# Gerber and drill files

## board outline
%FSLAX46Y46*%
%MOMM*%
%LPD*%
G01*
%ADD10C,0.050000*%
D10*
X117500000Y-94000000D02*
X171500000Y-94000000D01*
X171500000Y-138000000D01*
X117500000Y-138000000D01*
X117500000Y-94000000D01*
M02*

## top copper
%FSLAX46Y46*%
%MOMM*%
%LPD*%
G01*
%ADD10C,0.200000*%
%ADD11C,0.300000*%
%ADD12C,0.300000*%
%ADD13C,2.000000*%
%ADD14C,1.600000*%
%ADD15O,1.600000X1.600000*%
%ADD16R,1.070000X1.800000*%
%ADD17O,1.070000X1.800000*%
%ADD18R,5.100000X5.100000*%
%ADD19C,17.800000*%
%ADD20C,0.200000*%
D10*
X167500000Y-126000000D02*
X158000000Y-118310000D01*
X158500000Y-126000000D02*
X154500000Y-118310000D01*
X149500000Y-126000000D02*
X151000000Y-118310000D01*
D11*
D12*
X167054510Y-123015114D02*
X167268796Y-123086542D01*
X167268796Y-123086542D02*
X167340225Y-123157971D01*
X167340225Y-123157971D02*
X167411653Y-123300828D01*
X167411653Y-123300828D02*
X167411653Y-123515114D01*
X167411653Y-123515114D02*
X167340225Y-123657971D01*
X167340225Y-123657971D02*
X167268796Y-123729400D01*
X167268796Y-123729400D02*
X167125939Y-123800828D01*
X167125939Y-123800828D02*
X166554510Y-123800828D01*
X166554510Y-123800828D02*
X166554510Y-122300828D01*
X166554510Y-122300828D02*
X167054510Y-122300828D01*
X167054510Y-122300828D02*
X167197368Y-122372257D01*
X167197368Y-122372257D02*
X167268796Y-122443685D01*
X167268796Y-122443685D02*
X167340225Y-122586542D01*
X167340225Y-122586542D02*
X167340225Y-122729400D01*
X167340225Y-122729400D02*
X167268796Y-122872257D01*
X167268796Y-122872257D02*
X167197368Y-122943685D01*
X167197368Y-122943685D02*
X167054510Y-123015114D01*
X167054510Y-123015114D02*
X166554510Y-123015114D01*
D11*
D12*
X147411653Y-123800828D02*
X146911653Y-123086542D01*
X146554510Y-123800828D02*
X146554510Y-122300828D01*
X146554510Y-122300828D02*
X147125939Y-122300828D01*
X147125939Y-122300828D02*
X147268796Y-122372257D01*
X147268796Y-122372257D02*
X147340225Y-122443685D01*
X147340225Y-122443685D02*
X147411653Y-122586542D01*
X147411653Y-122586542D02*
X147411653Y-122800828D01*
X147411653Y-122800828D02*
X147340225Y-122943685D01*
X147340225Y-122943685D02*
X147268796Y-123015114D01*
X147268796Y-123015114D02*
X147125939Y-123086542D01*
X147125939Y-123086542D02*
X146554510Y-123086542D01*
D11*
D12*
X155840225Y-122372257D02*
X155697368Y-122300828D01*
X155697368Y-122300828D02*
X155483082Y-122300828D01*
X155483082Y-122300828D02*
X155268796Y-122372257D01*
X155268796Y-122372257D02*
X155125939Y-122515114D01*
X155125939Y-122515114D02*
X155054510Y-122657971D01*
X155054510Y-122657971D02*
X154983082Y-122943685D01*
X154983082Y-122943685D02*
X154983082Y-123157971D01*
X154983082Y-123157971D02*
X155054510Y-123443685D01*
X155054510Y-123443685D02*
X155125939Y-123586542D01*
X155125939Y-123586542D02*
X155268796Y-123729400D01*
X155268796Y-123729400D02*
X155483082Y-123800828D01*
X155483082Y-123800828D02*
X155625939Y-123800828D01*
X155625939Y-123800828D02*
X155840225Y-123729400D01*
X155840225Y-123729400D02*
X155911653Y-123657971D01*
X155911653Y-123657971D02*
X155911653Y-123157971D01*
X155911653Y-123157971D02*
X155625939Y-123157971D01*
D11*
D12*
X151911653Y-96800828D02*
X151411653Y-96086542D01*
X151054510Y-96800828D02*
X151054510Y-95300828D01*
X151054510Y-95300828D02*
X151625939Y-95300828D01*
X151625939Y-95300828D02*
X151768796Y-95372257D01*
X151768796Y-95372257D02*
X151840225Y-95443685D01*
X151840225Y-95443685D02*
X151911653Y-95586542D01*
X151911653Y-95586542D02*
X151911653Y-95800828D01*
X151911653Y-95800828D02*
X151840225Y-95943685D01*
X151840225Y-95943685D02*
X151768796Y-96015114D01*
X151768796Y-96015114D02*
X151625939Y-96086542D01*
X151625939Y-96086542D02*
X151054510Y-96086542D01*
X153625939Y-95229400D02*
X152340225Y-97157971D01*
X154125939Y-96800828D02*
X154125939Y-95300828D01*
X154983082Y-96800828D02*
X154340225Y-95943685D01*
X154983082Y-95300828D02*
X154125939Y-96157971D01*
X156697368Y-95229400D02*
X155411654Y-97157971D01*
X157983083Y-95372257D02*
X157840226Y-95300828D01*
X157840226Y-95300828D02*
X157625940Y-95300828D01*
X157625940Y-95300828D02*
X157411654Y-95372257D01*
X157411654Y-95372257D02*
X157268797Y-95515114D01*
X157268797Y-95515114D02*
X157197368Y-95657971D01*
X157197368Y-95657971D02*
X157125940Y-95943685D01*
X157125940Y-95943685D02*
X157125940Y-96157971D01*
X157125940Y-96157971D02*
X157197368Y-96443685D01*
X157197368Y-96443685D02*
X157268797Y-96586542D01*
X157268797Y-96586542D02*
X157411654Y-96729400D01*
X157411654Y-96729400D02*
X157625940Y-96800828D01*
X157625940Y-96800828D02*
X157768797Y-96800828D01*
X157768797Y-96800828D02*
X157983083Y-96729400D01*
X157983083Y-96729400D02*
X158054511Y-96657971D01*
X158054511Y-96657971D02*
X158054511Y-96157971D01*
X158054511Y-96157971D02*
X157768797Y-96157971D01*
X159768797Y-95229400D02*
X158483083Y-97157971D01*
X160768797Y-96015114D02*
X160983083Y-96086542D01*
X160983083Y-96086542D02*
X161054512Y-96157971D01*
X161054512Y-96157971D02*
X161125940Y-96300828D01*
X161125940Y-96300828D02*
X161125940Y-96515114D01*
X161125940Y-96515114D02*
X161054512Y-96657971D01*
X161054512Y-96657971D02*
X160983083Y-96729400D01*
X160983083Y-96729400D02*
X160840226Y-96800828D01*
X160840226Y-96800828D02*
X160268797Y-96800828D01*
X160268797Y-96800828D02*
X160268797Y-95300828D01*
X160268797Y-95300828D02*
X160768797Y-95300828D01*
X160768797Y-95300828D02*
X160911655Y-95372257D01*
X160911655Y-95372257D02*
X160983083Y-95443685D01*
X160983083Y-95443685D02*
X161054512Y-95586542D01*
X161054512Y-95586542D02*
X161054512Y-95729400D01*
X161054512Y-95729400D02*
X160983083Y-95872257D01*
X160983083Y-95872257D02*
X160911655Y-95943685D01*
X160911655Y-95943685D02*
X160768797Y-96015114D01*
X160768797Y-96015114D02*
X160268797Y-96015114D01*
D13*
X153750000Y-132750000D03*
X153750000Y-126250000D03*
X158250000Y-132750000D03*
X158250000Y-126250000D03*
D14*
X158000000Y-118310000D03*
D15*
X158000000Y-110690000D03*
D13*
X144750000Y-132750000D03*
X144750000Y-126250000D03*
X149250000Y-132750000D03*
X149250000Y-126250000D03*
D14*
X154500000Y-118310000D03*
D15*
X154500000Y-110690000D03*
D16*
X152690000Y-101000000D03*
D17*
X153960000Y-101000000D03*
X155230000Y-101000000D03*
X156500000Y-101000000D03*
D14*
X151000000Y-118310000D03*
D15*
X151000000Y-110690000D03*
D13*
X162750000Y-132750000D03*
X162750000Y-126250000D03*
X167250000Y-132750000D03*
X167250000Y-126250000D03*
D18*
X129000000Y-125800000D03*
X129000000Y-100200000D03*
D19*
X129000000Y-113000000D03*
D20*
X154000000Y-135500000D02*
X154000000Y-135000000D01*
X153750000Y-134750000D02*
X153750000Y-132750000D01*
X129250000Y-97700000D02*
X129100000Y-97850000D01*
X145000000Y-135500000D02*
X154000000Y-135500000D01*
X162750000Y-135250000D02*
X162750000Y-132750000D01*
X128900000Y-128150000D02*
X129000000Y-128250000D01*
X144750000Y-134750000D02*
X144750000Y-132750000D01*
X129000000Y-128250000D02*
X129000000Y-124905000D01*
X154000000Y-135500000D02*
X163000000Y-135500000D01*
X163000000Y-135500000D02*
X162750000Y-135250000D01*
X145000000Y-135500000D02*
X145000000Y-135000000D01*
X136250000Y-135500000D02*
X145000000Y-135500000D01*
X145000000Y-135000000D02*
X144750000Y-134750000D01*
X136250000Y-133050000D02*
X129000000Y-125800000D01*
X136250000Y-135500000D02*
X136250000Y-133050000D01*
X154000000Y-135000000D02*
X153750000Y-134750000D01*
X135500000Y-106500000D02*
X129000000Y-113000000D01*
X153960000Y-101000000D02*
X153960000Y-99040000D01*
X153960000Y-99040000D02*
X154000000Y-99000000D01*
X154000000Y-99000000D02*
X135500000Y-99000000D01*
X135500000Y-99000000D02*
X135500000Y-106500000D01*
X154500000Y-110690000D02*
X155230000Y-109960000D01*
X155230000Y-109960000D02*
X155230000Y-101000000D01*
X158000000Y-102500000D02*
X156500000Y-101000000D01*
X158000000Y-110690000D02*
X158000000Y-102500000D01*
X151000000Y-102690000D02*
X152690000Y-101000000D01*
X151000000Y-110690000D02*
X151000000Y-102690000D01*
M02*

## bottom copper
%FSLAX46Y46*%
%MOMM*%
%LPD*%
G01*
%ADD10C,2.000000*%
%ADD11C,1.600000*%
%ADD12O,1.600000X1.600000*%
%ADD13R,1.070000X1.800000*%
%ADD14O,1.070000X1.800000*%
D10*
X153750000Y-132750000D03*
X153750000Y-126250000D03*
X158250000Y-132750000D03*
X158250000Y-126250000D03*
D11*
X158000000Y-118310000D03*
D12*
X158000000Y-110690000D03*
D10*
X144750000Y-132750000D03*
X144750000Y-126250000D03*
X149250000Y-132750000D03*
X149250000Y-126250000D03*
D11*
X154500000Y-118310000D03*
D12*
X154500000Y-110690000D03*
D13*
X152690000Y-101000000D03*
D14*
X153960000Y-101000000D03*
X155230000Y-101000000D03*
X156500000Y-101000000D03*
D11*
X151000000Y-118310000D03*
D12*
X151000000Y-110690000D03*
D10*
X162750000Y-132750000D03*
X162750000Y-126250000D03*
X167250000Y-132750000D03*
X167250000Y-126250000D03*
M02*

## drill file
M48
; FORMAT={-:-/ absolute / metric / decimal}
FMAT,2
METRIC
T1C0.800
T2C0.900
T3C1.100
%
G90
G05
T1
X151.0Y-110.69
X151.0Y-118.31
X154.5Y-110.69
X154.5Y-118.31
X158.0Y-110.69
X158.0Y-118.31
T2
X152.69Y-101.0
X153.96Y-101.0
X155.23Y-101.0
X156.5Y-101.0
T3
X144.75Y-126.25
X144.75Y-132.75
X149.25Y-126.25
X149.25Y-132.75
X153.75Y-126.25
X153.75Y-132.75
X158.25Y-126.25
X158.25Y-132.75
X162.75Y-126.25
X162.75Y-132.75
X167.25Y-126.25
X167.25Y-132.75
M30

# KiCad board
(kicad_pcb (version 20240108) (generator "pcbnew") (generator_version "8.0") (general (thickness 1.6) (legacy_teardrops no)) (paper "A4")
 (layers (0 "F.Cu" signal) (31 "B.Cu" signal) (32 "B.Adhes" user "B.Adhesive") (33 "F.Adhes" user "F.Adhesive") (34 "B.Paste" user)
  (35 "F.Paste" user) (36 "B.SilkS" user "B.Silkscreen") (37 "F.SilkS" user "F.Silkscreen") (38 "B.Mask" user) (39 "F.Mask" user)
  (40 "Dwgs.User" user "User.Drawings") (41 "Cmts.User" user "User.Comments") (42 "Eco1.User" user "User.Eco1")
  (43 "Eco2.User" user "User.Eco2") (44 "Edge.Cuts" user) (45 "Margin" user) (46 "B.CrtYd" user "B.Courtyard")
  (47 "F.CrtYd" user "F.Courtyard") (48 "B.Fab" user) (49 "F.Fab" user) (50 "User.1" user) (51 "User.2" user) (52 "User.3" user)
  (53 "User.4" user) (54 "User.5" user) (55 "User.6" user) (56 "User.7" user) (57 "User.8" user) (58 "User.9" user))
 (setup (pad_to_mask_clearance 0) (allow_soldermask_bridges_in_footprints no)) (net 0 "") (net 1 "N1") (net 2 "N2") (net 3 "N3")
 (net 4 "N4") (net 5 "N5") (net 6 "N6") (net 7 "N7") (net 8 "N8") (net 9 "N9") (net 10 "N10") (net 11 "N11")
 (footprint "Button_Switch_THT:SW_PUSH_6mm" (layer "F.Cu") (at 153.75 132.75 90)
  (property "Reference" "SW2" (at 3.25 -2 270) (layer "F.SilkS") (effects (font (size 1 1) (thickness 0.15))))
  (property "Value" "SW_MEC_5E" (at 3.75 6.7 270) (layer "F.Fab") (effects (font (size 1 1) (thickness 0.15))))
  (pad "1" thru_hole circle (at 0 0 180) (size 2 2) (drill 1.1) (layers "*.Cu" "*.Mask") (remove_unused_layers no) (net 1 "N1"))
  (pad "1" thru_hole circle (at 6.5 0 180) (size 2 2) (drill 1.1) (layers "*.Cu" "*.Mask") (remove_unused_layers no) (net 1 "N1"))
  (pad "2" thru_hole circle (at 0 4.5 180) (size 2 2) (drill 1.1) (layers "*.Cu" "*.Mask") (remove_unused_layers no) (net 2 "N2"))
  (pad "2" thru_hole circle (at 6.5 4.5 180) (size 2 2) (drill 1.1) (layers "*.Cu" "*.Mask") (remove_unused_layers no) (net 2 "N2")))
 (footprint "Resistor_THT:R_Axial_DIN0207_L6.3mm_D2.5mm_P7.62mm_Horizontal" (layer "F.Cu") (at 158 118.31 90)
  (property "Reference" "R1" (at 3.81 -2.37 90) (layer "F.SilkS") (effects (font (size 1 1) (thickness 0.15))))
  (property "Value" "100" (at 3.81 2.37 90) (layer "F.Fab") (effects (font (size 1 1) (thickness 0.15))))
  (pad "1" thru_hole circle (at 0 0 90) (size 1.6 1.6) (drill 0.8) (layers "*.Cu" "*.Mask") (remove_unused_layers no) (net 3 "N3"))
  (pad "2" thru_hole oval (at 7.62 0 90) (size 1.6 1.6) (drill 0.8) (layers "*.Cu" "*.Mask") (remove_unused_layers no) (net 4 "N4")))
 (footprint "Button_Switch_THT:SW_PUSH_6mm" (layer "F.Cu") (at 144.75 132.75 90)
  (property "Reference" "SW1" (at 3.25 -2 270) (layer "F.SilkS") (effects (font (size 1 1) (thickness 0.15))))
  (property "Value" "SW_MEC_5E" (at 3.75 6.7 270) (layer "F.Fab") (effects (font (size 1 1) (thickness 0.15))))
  (pad "1" thru_hole circle (at 0 0 180) (size 2 2) (drill 1.1) (layers "*.Cu" "*.Mask") (remove_unused_layers no) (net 1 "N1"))
  (pad "1" thru_hole circle (at 6.5 0 180) (size 2 2) (drill 1.1) (layers "*.Cu" "*.Mask") (remove_unused_layers no) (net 1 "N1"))
  (pad "2" thru_hole circle (at 0 4.5 180) (size 2 2) (drill 1.1) (layers "*.Cu" "*.Mask") (remove_unused_layers no) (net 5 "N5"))
  (pad "2" thru_hole circle (at 6.5 4.5 180) (size 2 2) (drill 1.1) (layers "*.Cu" "*.Mask") (remove_unused_layers no) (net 5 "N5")))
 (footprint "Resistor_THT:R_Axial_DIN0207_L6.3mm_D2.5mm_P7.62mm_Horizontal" (layer "F.Cu") (at 154.5 118.31 90)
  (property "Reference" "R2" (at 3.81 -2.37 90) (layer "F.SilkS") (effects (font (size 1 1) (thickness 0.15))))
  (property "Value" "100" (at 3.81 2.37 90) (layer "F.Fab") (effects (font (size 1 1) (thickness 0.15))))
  (pad "1" thru_hole circle (at 0 0 90) (size 1.6 1.6) (drill 0.8) (layers "*.Cu" "*.Mask") (remove_unused_layers no) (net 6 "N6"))
  (pad "2" thru_hole oval (at 7.62 0 90) (size 1.6 1.6) (drill 0.8) (layers "*.Cu" "*.Mask") (remove_unused_layers no) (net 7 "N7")))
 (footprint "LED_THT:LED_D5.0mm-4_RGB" (layer "F.Cu") (at 152.69 101)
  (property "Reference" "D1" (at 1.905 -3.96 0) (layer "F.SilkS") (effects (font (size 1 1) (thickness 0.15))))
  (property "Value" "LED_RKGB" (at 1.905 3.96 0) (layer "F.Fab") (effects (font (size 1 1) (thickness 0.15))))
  (pad "1" thru_hole rect (at 0 0) (size 1.07 1.8) (drill 0.9) (layers "*.Cu" "*.Mask") (remove_unused_layers no) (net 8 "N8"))
  (pad "2" thru_hole oval (at 1.27 0) (size 1.07 1.8) (drill 0.9) (layers "*.Cu" "*.Mask") (remove_unused_layers no) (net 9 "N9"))
  (pad "3" thru_hole oval (at 2.54 0) (size 1.07 1.8) (drill 0.9) (layers "*.Cu" "*.Mask") (remove_unused_layers no) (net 7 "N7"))
  (pad "4" thru_hole oval (at 3.81 0) (size 1.07 1.8) (drill 0.9) (layers "*.Cu" "*.Mask") (remove_unused_layers no) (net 4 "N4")))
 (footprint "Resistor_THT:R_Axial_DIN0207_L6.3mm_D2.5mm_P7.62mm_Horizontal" (layer "F.Cu") (at 151 118.31 90)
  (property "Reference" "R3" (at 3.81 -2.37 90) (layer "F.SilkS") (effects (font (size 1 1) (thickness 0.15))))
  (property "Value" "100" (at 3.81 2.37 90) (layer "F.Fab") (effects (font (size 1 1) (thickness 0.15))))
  (pad "1" thru_hole circle (at 0 0 90) (size 1.6 1.6) (drill 0.8) (layers "*.Cu" "*.Mask") (remove_unused_layers no) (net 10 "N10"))
  (pad "2" thru_hole oval (at 7.62 0 90) (size 1.6 1.6) (drill 0.8) (layers "*.Cu" "*.Mask") (remove_unused_layers no) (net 8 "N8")))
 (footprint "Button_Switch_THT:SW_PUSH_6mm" (layer "F.Cu") (at 162.75 132.75 90)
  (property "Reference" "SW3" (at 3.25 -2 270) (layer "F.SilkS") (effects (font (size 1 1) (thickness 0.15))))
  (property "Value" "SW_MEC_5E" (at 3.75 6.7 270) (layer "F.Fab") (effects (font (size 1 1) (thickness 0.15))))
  (pad "1" thru_hole circle (at 0 0 180) (size 2 2) (drill 1.1) (layers "*.Cu" "*.Mask") (remove_unused_layers no) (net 1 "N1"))
  (pad "1" thru_hole circle (at 6.5 0 180) (size 2 2) (drill 1.1) (layers "*.Cu" "*.Mask") (remove_unused_layers no) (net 1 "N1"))
  (pad "2" thru_hole circle (at 0 4.5 180) (size 2 2) (drill 1.1) (layers "*.Cu" "*.Mask") (remove_unused_layers no) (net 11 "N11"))
  (pad "2" thru_hole circle (at 6.5 4.5 180) (size 2 2) (drill 1.1) (layers "*.Cu" "*.Mask") (remove_unused_layers no) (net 11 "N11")))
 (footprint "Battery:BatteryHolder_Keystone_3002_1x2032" (layer "F.Cu") (at 129 113 90)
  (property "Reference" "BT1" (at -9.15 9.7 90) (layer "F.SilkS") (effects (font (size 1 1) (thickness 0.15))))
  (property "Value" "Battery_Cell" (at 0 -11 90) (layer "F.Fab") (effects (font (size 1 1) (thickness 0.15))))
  (pad "1" smd rect (at -12.8 0 90) (size 5.1 5.1) (layers "F.Cu" "F.Paste" "F.Mask") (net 1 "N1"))
  (pad "1" smd rect (at 12.8 0 90) (size 5.1 5.1) (layers "F.Cu" "F.Paste" "F.Mask") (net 1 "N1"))
  (pad "2" smd circle (at 0 0 90) (size 17.8 17.8) (layers "F.Cu" "F.Mask") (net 9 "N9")))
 (gr_line (start 167.5 126) (end 158 118.31) (stroke (width 0.2) (type default)) (layer "F.Cu"))
 (gr_line (start 158.5 126) (end 154.5 118.31) (stroke (width 0.2) (type default)) (layer "F.Cu"))
 (gr_line (start 149.5 126) (end 151 118.31) (stroke (width 0.2) (type default)) (layer "F.Cu"))
 (gr_rect (start 117.5 94) (end 171.5 138) (stroke (width 0.05) (type default)) (fill none) (layer "Edge.Cuts"))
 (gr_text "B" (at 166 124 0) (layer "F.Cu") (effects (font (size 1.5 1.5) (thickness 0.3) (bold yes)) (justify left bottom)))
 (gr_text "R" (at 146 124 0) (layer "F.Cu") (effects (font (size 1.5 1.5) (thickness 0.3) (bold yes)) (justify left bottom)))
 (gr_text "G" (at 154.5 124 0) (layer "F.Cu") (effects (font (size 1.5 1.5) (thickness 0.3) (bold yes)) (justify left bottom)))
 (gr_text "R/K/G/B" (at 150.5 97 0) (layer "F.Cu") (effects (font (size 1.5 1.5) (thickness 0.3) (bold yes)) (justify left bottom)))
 (segment (start 154 135.5) (end 154 135) (width 0.2) (layer "F.Cu") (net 1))
 (segment (start 153.75 134.75) (end 153.75 132.75) (width 0.2) (layer "F.Cu") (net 1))
 (segment (start 129.25 97.7) (end 129.1 97.85) (width 0.2) (layer "F.Cu") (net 1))
 (segment (start 145 135.5) (end 154 135.5) (width 0.2) (layer "F.Cu") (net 1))
 (segment (start 162.75 135.25) (end 162.75 132.75) (width 0.2) (layer "F.Cu") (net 1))
 (segment (start 128.9 128.15) (end 129 128.25) (width 0.2) (layer "F.Cu") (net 1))
 (segment (start 144.75 134.75) (end 144.75 132.75) (width 0.2) (layer "F.Cu") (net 1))
 (segment (start 129 128.25) (end 129 124.905) (width 0.2) (layer "F.Cu") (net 1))
 (segment (start 154 135.5) (end 163 135.5) (width 0.2) (layer "F.Cu") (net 1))
 (segment (start 163 135.5) (end 162.75 135.25) (width 0.2) (layer "F.Cu") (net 1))
 (segment (start 145 135.5) (end 145 135) (width 0.2) (layer "F.Cu") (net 1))
 (segment (start 136.25 135.5) (end 145 135.5) (width 0.2) (layer "F.Cu") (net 1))
 (segment (start 145 135) (end 144.75 134.75) (width 0.2) (layer "F.Cu") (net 1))
 (segment (start 136.25 133.05) (end 129 125.8) (width 0.2) (layer "F.Cu") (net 1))
 (segment (start 136.25 135.5) (end 136.25 133.05) (width 0.2) (layer "F.Cu") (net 1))
 (segment (start 154 135) (end 153.75 134.75) (width 0.2) (layer "F.Cu") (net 1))
 (segment (start 135.5 106.5) (end 129 113) (width 0.2) (layer "F.Cu") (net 9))
 (segment (start 153.96 101) (end 153.96 99.04) (width 0.2) (layer "F.Cu") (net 9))
 (segment (start 153.96 99.04) (end 154 99) (width 0.2) (layer "F.Cu") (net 9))
 (segment (start 154 99) (end 135.5 99) (width 0.2) (layer "F.Cu") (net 9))
 (segment (start 135.5 99) (end 135.5 106.5) (width 0.2) (layer "F.Cu") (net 9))
 (segment (start 154.5 110.69) (end 155.23 109.96) (width 0.2) (layer "F.Cu") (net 7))
 (segment (start 155.23 109.96) (end 155.23 101) (width 0.2) (layer "F.Cu") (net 7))
 (segment (start 158 102.5) (end 156.5 101) (width 0.2) (layer "F.Cu") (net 4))
 (segment (start 158 110.69) (end 158 102.5) (width 0.2) (layer "F.Cu") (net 4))
 (segment (start 151 102.69) (end 152.69 101) (width 0.2) (layer "F.Cu") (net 8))
 (segment (start 151 110.69) (end 151 102.69) (width 0.2) (layer "F.Cu") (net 8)))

